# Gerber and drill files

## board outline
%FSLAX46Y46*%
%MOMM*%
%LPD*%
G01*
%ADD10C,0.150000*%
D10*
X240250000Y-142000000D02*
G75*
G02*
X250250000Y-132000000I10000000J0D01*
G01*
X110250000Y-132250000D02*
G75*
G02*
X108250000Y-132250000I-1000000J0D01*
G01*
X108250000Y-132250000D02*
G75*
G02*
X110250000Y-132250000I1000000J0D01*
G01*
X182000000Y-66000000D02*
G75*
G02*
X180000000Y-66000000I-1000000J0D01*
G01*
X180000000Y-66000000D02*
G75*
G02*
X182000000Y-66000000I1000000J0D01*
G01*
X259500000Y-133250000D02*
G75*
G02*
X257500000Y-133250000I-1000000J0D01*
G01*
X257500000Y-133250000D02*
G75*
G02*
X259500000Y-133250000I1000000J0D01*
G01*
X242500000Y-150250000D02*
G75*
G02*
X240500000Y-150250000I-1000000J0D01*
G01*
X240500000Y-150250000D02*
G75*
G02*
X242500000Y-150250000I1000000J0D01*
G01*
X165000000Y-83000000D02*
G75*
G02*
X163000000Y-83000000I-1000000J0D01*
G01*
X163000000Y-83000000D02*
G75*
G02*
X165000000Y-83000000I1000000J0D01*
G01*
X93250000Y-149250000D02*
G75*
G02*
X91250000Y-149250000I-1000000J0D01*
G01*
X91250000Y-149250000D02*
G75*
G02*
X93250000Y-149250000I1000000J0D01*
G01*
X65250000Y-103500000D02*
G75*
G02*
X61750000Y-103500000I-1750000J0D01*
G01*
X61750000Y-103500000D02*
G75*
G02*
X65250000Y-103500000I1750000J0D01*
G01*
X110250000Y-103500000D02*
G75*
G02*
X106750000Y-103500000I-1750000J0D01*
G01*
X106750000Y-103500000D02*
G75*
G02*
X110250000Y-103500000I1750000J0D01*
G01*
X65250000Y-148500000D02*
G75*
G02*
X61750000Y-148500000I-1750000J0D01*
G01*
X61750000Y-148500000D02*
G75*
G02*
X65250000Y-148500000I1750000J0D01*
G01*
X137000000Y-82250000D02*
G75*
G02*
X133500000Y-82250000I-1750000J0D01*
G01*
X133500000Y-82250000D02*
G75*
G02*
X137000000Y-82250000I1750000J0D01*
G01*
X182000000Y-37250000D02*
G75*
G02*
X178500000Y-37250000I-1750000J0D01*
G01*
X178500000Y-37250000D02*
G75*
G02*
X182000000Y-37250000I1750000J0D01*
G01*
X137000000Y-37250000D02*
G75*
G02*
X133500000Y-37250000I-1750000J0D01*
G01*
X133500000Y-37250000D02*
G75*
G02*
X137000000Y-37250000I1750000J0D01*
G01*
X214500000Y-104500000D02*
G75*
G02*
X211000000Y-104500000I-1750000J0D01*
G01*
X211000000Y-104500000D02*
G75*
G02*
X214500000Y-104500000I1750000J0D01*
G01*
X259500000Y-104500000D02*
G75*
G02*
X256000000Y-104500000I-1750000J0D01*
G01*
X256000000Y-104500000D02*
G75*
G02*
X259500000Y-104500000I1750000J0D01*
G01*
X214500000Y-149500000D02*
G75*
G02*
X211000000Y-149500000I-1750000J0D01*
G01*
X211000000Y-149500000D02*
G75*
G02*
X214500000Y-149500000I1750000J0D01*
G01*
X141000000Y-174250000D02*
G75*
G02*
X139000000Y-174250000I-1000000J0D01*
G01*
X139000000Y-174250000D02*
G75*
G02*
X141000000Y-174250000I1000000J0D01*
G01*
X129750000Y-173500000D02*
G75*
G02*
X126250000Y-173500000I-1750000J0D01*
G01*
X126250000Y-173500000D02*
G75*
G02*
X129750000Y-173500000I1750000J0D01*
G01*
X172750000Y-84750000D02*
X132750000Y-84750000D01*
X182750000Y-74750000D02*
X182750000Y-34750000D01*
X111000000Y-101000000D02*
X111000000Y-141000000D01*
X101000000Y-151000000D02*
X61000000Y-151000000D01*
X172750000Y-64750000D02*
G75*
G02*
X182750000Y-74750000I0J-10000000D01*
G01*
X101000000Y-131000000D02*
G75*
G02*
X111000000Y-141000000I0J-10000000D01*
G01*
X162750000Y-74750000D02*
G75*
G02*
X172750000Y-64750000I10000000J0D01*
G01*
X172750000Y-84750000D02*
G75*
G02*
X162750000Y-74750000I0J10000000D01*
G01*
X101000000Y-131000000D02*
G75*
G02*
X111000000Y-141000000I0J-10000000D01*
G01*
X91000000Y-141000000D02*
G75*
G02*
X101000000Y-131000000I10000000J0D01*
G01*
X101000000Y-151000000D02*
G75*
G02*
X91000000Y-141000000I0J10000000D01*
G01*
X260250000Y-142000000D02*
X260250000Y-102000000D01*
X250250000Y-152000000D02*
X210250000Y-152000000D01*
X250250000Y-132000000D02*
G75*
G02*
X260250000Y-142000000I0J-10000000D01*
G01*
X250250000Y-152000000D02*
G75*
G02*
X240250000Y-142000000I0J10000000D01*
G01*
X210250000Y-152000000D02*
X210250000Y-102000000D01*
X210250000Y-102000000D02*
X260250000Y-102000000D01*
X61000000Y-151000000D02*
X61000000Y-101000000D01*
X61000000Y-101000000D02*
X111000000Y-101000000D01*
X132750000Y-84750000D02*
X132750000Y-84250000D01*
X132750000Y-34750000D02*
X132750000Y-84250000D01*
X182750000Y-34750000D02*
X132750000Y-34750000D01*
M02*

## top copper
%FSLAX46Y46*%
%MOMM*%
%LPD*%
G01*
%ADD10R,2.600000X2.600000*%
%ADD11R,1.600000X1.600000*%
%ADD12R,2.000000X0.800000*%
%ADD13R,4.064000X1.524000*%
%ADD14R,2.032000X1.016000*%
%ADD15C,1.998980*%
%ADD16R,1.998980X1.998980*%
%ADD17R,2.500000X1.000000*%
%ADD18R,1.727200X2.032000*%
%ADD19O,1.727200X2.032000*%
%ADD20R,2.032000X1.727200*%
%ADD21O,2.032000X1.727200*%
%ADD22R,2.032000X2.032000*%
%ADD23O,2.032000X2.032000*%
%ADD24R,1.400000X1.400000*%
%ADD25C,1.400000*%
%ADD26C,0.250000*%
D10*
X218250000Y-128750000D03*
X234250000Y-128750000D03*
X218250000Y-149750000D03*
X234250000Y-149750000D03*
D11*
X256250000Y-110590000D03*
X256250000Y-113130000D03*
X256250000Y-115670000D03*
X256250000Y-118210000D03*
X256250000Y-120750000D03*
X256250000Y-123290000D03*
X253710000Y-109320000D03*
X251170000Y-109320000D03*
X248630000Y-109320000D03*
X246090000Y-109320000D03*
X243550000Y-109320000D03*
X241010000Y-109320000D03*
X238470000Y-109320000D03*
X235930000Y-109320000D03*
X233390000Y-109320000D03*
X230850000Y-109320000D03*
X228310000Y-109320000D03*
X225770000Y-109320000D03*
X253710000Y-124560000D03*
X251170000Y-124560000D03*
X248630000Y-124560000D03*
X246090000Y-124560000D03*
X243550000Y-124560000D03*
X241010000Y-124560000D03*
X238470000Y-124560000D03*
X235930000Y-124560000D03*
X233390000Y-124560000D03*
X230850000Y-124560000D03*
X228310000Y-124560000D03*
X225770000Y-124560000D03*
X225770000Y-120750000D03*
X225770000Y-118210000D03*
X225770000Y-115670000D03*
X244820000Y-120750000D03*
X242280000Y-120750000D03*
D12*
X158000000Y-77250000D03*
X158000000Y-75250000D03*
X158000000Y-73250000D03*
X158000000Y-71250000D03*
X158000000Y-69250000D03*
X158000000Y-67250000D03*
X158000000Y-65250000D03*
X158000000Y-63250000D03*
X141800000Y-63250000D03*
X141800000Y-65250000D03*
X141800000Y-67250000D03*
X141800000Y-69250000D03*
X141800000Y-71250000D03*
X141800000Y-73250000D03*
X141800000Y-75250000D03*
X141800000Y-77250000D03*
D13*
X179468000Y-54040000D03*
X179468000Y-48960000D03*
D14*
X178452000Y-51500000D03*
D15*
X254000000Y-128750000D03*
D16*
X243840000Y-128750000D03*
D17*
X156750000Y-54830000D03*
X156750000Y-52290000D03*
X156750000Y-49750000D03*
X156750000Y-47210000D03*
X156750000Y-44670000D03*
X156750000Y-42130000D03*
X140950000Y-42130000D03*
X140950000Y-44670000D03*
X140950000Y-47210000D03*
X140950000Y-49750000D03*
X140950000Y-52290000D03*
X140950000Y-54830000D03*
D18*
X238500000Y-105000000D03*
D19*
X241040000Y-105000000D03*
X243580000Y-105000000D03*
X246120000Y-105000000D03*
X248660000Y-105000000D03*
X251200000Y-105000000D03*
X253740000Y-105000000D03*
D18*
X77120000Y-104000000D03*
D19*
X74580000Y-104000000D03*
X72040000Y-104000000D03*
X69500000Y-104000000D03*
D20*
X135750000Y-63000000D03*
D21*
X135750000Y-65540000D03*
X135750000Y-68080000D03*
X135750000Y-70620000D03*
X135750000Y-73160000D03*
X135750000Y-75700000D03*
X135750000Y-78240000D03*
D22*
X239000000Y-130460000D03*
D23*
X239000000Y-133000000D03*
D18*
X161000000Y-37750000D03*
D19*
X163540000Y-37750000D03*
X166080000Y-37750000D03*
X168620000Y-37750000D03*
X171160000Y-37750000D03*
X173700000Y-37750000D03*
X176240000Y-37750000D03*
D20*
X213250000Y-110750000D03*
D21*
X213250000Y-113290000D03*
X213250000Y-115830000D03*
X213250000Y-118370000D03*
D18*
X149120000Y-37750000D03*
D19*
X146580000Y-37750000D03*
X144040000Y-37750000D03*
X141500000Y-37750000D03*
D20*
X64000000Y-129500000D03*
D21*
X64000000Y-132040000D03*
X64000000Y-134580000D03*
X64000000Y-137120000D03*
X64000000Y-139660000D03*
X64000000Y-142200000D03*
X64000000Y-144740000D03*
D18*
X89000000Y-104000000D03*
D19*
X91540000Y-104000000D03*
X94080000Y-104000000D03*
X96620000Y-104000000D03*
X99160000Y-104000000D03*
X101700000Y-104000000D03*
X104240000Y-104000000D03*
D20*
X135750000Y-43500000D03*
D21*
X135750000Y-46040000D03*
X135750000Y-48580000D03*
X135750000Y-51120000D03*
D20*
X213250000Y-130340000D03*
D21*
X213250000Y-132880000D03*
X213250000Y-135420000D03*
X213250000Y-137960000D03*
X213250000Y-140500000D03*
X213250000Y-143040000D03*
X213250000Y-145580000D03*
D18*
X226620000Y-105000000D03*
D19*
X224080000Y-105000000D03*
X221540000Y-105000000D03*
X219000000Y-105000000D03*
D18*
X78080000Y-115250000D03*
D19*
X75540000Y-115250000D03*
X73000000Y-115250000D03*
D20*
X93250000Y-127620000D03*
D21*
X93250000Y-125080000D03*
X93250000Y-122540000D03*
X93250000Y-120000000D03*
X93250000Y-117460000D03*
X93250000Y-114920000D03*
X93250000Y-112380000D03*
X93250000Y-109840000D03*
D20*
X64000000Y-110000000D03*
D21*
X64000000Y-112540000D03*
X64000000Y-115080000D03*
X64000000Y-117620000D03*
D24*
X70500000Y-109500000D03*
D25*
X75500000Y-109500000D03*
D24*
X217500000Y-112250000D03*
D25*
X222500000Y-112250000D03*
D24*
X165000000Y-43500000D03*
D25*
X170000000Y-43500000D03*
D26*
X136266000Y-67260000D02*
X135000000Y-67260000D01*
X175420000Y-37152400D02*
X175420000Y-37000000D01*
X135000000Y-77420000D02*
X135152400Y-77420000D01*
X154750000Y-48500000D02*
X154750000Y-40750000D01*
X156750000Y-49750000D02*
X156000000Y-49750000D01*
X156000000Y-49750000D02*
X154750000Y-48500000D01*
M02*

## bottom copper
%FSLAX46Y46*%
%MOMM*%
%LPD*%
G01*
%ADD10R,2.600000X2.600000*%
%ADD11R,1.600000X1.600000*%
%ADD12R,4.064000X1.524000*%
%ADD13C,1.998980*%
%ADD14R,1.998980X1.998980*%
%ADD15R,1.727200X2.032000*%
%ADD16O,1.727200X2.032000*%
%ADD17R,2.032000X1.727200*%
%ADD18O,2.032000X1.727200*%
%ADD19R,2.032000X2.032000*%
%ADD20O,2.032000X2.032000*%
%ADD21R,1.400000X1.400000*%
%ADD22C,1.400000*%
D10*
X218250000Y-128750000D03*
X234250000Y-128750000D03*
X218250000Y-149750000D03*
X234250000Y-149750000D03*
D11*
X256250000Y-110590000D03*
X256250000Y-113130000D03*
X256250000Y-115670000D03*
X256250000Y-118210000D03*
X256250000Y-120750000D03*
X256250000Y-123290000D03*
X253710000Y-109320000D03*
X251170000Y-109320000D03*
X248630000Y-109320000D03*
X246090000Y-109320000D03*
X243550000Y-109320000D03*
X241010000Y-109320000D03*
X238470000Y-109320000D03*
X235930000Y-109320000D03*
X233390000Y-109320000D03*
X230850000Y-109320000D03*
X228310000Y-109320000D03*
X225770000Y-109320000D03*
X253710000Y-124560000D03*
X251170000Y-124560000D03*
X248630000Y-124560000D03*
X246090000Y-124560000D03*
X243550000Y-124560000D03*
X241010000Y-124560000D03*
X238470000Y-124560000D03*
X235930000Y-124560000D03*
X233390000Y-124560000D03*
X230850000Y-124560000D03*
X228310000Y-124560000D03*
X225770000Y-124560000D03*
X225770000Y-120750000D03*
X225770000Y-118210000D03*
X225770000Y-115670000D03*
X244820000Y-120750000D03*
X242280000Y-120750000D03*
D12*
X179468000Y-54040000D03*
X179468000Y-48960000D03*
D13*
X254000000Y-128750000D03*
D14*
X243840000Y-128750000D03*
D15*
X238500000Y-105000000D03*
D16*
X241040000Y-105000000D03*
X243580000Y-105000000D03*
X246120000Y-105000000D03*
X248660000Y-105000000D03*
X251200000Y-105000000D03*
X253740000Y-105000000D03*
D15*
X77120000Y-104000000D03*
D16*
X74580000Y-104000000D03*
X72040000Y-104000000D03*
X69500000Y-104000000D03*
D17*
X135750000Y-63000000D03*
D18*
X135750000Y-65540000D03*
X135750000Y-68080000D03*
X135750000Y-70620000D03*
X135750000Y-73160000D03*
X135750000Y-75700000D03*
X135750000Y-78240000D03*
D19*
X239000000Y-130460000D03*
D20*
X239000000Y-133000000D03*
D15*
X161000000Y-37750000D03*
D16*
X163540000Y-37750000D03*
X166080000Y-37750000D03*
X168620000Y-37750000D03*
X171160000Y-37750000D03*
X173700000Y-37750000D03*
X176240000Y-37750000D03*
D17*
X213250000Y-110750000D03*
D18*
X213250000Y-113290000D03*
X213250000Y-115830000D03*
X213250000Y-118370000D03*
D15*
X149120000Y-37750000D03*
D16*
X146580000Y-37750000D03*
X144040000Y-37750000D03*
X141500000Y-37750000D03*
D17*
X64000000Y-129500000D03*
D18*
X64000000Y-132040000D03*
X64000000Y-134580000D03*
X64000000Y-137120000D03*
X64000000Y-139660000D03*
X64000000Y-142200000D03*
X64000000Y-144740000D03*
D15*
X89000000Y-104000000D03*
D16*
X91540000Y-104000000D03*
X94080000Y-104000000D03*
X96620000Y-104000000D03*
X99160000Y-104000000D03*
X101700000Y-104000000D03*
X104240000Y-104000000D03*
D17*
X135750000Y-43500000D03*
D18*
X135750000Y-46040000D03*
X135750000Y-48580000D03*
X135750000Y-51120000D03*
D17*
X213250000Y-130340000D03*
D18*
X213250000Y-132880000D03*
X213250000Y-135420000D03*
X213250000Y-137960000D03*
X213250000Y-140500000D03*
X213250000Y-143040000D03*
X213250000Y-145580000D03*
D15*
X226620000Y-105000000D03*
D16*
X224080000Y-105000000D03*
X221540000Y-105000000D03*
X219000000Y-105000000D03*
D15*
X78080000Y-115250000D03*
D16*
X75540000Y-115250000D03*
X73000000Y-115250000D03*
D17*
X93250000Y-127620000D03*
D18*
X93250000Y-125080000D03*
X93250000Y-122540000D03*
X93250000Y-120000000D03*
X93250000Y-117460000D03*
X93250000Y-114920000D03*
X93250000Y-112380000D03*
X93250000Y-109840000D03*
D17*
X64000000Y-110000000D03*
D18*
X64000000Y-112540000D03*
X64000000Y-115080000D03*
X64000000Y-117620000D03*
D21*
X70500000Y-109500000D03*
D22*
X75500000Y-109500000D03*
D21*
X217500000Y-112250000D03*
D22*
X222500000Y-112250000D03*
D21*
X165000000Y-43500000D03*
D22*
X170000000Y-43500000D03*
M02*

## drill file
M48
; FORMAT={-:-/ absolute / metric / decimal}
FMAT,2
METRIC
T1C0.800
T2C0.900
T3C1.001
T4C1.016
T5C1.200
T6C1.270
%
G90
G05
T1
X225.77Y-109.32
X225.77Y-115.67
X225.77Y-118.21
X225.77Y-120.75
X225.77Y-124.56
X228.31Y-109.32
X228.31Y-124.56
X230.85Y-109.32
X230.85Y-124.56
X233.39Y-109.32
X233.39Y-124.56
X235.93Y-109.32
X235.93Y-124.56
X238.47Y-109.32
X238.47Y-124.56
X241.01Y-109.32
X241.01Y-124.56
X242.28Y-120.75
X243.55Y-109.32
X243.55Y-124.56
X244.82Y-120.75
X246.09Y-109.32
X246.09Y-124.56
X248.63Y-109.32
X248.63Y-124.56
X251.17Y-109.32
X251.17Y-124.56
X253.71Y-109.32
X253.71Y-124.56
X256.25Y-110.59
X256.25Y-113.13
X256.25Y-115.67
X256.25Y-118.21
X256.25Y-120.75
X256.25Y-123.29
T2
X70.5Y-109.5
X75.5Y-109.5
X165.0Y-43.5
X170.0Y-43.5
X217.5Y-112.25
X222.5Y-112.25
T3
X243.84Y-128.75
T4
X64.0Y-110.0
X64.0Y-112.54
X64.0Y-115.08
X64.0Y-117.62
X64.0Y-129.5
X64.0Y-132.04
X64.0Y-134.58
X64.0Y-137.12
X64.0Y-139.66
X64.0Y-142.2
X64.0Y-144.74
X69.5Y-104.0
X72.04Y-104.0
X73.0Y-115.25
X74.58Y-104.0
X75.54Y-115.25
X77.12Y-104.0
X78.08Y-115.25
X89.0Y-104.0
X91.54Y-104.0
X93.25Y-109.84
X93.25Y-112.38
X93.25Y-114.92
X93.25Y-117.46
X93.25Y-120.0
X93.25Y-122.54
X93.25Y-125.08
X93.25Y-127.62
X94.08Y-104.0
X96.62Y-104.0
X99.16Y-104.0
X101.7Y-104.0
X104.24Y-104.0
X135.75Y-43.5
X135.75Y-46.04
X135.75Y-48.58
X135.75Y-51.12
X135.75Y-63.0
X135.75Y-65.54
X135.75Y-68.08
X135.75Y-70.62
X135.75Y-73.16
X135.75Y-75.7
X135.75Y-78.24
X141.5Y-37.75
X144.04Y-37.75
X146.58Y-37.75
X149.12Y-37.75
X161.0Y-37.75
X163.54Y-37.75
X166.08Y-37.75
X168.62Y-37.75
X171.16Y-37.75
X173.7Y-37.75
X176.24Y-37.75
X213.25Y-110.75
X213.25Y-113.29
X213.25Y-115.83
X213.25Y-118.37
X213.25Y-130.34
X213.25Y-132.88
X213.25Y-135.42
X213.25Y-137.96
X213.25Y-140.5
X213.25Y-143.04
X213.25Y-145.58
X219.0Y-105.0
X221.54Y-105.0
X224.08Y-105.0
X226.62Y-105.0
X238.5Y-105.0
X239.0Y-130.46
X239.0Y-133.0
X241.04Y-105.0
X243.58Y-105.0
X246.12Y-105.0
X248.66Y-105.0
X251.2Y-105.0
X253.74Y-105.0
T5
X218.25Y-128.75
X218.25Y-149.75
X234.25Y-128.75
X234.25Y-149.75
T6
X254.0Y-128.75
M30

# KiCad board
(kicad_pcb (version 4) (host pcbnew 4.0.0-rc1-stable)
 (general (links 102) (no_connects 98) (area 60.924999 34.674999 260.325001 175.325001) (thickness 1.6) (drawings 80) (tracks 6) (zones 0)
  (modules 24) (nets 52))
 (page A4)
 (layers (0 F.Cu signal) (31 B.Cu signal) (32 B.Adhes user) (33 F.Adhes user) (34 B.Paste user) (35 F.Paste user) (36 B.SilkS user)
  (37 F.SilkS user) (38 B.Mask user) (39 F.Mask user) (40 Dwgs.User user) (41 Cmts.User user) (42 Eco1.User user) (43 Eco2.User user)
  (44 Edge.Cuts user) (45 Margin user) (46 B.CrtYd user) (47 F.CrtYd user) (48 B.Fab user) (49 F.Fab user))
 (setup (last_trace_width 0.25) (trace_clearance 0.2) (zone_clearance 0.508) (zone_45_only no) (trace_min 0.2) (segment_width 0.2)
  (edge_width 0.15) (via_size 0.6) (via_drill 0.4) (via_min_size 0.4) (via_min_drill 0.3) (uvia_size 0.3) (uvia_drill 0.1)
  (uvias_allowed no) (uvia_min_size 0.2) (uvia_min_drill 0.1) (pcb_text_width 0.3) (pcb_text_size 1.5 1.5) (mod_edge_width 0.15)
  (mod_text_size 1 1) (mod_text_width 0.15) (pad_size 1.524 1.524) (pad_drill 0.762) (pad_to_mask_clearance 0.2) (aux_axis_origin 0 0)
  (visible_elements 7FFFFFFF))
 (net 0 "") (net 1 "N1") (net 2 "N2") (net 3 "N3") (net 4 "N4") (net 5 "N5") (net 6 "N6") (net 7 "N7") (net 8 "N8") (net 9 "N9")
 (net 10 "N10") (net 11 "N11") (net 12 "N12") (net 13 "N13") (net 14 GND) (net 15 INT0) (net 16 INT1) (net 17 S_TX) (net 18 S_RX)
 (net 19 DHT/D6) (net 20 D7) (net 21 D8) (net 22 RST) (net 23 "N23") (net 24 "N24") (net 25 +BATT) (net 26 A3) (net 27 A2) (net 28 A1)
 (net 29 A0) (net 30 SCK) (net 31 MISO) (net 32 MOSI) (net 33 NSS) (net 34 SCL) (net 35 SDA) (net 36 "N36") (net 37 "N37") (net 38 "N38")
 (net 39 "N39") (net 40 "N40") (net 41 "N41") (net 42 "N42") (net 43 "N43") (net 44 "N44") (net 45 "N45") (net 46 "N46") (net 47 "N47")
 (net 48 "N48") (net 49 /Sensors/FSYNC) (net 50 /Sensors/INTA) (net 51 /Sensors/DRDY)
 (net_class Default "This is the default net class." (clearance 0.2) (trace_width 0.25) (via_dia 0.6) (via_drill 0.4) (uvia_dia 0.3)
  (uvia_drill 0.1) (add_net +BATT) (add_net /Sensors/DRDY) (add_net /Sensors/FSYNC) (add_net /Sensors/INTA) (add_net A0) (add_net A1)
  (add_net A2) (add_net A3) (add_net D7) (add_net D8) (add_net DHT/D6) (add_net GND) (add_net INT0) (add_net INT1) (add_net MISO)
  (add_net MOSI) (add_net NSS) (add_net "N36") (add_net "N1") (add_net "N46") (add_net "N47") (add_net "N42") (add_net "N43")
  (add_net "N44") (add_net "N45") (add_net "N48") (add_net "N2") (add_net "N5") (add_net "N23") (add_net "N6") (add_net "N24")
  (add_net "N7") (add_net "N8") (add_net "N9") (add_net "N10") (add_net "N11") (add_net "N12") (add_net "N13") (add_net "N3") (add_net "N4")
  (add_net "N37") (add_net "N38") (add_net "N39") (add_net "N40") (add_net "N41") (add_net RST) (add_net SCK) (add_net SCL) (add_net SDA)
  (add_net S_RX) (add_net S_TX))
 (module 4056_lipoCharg (layer F.Cu) (at 215.5 125.5)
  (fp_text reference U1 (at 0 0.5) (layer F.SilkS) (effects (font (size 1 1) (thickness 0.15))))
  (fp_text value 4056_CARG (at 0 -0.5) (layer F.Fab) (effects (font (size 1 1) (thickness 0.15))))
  (pad 3 thru_hole rect (at 2.75 3.25) (size 2.6 2.6) (drill 1.2) (layers *.Cu *.Mask F.SilkS) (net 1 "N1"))
  (pad 4 thru_hole rect (at 18.75 3.25) (size 2.6 2.6) (drill 1.2) (layers *.Cu *.Mask F.SilkS) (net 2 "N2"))
  (pad 1 thru_hole rect (at 2.75 24.25) (size 2.6 2.6) (drill 1.2) (layers *.Cu *.Mask F.SilkS) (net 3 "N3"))
  (pad 2 thru_hole rect (at 18.75 24.25) (size 2.6 2.6) (drill 1.2) (layers *.Cu *.Mask F.SilkS) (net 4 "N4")))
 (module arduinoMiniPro (layer F.Cu) (at 247.36 114.4 270)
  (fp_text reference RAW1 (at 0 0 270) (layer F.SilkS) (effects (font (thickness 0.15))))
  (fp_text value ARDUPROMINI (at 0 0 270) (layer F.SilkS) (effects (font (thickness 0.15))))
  (pad 1 thru_hole rect (at -3.81 -8.89) (size 1.6 1.6) (drill 0.8) (layers *.Cu *.Mask) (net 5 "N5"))
  (pad 2 thru_hole rect (at -1.27 -8.89) (size 1.6 1.6) (drill 0.8) (layers *.Cu *.Mask) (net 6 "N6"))
  (pad 3 thru_hole rect (at 1.27 -8.89) (size 1.6 1.6) (drill 0.8) (layers *.Cu *.Mask) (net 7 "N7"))
  (pad 4 thru_hole rect (at 3.81 -8.89) (size 1.6 1.6) (drill 0.8) (layers *.Cu *.Mask) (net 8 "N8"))
  (pad 5 thru_hole rect (at 6.35 -8.89) (size 1.6 1.6) (drill 0.8) (layers *.Cu *.Mask) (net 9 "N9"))
  (pad 6 thru_hole rect (at 8.89 -8.89) (size 1.6 1.6) (drill 0.8) (layers *.Cu *.Mask) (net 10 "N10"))
  (pad 7 thru_hole rect (at -5.08 -6.35 90) (size 1.6 1.6) (drill 0.8) (layers *.Cu *.Mask) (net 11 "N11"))
  (pad 8 thru_hole rect (at -5.08 -3.81 90) (size 1.6 1.6) (drill 0.8) (layers *.Cu *.Mask) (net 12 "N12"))
  (pad 9 thru_hole rect (at -5.08 -1.27 90) (size 1.6 1.6) (drill 0.8) (layers *.Cu *.Mask) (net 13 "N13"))
  (pad 10 thru_hole rect (at -5.08 1.27 90) (size 1.6 1.6) (drill 0.8) (layers *.Cu *.Mask) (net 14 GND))
  (pad 11 thru_hole rect (at -5.08 3.81 90) (size 1.6 1.6) (drill 0.8) (layers *.Cu *.Mask) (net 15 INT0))
  (pad 12 thru_hole rect (at -5.08 6.35 90) (size 1.6 1.6) (drill 0.8) (layers *.Cu *.Mask) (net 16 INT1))
  (pad 13 thru_hole rect (at -5.08 8.89 90) (size 1.6 1.6) (drill 0.8) (layers *.Cu *.Mask) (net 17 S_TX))
  (pad 14 thru_hole rect (at -5.08 11.43 90) (size 1.6 1.6) (drill 0.8) (layers *.Cu *.Mask) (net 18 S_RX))
  (pad 15 thru_hole rect (at -5.08 13.97 90) (size 1.6 1.6) (drill 0.8) (layers *.Cu *.Mask) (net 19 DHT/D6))
  (pad 16 thru_hole rect (at -5.08 16.51 90) (size 1.6 1.6) (drill 0.8) (layers *.Cu *.Mask) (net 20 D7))
  (pad 17 thru_hole rect (at -5.08 19.05 90) (size 1.6 1.6) (drill 0.8) (layers *.Cu *.Mask) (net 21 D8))
  (pad 18 thru_hole rect (at -5.08 21.59 90) (size 1.6 1.6) (drill 0.8) (layers *.Cu *.Mask) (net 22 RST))
  (pad 19 thru_hole rect (at 10.16 -6.35 90) (size 1.6 1.6) (drill 0.8) (layers *.Cu *.Mask) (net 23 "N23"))
  (pad 20 thru_hole rect (at 10.16 -3.81 90) (size 1.6 1.6) (drill 0.8) (layers *.Cu *.Mask) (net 14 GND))
  (pad 21 thru_hole rect (at 10.16 -1.27 90) (size 1.6 1.6) (drill 0.8) (layers *.Cu *.Mask) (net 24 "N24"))
  (pad 22 thru_hole rect (at 10.16 1.27 90) (size 1.6 1.6) (drill 0.8) (layers *.Cu *.Mask) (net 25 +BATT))
  (pad 23 thru_hole rect (at 10.16 3.81 90) (size 1.6 1.6) (drill 0.8) (layers *.Cu *.Mask) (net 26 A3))
  (pad 24 thru_hole rect (at 10.16 6.35 90) (size 1.6 1.6) (drill 0.8) (layers *.Cu *.Mask) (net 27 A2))
  (pad 25 thru_hole rect (at 10.16 8.89 90) (size 1.6 1.6) (drill 0.8) (layers *.Cu *.Mask) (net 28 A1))
  (pad 26 thru_hole rect (at 10.16 11.43 90) (size 1.6 1.6) (drill 0.8) (layers *.Cu *.Mask) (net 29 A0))
  (pad 27 thru_hole rect (at 10.16 13.97 90) (size 1.6 1.6) (drill 0.8) (layers *.Cu *.Mask) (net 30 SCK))
  (pad 28 thru_hole rect (at 10.16 16.51 90) (size 1.6 1.6) (drill 0.8) (layers *.Cu *.Mask) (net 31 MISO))
  (pad 29 thru_hole rect (at 10.16 19.05 90) (size 1.6 1.6) (drill 0.8) (layers *.Cu *.Mask) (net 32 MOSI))
  (pad 30 thru_hole rect (at 10.16 21.59 90) (size 1.6 1.6) (drill 0.8) (layers *.Cu *.Mask) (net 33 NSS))
  (pad A7 thru_hole rect (at 6.35 21.59 180) (size 1.6 1.6) (drill 0.8) (layers *.Cu *.Mask))
  (pad A6 thru_hole rect (at 3.81 21.59 180) (size 1.6 1.6) (drill 0.8) (layers *.Cu *.Mask))
  (pad GND4 thru_hole rect (at 1.27 21.59 180) (size 1.6 1.6) (drill 0.8) (layers *.Cu *.Mask))
  (pad 32 thru_hole rect (at 6.35 2.54 180) (size 1.6 1.6) (drill 0.8) (layers *.Cu *.Mask) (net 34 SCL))
  (pad 31 thru_hole rect (at 6.35 5.08 180) (size 1.6 1.6) (drill 0.8) (layers *.Cu *.Mask) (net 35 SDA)))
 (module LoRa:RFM (layer F.Cu) (at 149.9 70.25)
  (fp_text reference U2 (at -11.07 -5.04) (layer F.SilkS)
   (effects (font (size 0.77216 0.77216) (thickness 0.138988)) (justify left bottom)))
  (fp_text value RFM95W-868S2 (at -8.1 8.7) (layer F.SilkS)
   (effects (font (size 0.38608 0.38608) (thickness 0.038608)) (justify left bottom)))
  (pad 9 smd rect (at 8.1 7 180) (size 2 0.8) (layers F.Cu F.Paste F.Mask) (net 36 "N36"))
  (pad 10 smd rect (at 8.1 5 180) (size 2 0.8) (layers F.Cu F.Paste F.Mask) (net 14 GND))
  (pad 11 smd rect (at 8.1 3 180) (size 2 0.8) (layers F.Cu F.Paste F.Mask) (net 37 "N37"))
  (pad 12 smd rect (at 8.1 1 180) (size 2 0.8) (layers F.Cu F.Paste F.Mask) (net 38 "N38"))
  (pad 13 smd rect (at 8.1 -1 180) (size 2 0.8) (layers F.Cu F.Paste F.Mask) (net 25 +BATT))
  (pad 14 smd rect (at 8.1 -3 180) (size 2 0.8) (layers F.Cu F.Paste F.Mask) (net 15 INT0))
  (pad 15 smd rect (at 8.1 -5 180) (size 2 0.8) (layers F.Cu F.Paste F.Mask) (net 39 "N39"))
  (pad 16 smd rect (at 8.1 -7 180) (size 2 0.8) (layers F.Cu F.Paste F.Mask) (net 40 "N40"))
  (pad 1 smd rect (at -8.1 -7) (size 2 0.8) (layers F.Cu F.Paste F.Mask) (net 14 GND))
  (pad 2 smd rect (at -8.1 -5) (size 2 0.8) (layers F.Cu F.Paste F.Mask) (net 31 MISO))
  (pad 3 smd rect (at -8.1 -3) (size 2 0.8) (layers F.Cu F.Paste F.Mask) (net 32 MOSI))
  (pad 4 smd rect (at -8.1 -1) (size 2 0.8) (layers F.Cu F.Paste F.Mask) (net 30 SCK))
  (pad 5 smd rect (at -8.1 1) (size 2 0.8) (layers F.Cu F.Paste F.Mask) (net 33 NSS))
  (pad 6 smd rect (at -8.1 3) (size 2 0.8) (layers F.Cu F.Paste F.Mask) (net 22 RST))
  (pad 7 smd rect (at -8.1 5) (size 2 0.8) (layers F.Cu F.Paste F.Mask) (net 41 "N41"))
  (pad 8 smd rect (at -8.1 7 180) (size 2 0.8) (layers F.Cu F.Paste F.Mask) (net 14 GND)))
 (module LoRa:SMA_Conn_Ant (layer F.Cu) (at 181.5 51.5 180)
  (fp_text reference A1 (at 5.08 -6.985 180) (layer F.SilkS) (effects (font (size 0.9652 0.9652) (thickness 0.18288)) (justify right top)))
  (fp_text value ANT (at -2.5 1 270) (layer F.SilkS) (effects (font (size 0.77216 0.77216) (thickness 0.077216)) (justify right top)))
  (pad 1 smd rect (at 2.032 -2.54 270) (size 1.524 4.064) (layers F.Cu F.Paste F.Mask) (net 14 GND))
  (pad 3 smd rect (at 2.032 2.54 270) (size 1.524 4.064) (layers F.Cu F.Paste F.Mask) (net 14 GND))
  (pad 2 smd rect (at 3.048 0 270) (size 1.016 2.032) (layers F.Cu F.Paste F.Mask) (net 36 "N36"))
  (pad "" smd rect (at 2.032 -2.54 270) (size 1.524 4.064) (layers B.Cu B.Paste B.Mask))
  (pad "" smd rect (at 2.032 2.54 270) (size 1.524 4.064) (layers B.Cu B.Paste B.Mask)))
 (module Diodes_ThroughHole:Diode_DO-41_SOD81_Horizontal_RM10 (layer F.Cu) (at 243.84 128.75254)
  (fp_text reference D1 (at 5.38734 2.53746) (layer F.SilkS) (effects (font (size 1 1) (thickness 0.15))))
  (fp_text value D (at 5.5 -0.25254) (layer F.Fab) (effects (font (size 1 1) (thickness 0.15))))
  (pad 2 thru_hole circle (at 10.16 -0.00254 180) (size 1.99898 1.99898) (drill 1.27) (layers *.Cu *.Mask F.SilkS) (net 1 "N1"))
  (pad 1 thru_hole rect (at 0 -0.00254 180) (size 1.99898 1.99898) (drill 1.00076) (layers *.Cu *.Mask F.SilkS) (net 25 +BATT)))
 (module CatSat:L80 (layer F.Cu) (at 148.883668 49.118506 180) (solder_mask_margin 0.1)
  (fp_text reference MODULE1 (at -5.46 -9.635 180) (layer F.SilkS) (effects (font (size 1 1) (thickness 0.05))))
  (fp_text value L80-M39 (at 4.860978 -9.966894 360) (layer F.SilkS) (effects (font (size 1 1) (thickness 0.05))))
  (pad 1 smd rect (at -7.866332 -5.711494) (size 2.5 1) (layers F.Cu F.Paste F.Mask) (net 17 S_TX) (solder_mask_margin 0.2))
  (pad 2 smd rect (at -7.866332 -3.171494) (size 2.5 1) (layers F.Cu F.Paste F.Mask) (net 18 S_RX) (solder_mask_margin 0.2))
  (pad 3 smd rect (at -7.866332 -0.631494) (size 2.5 1) (layers F.Cu F.Paste F.Mask) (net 14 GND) (solder_mask_margin 0.2))
  (pad 4 smd rect (at -7.866332 1.908506) (size 2.5 1) (layers F.Cu F.Paste F.Mask) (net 25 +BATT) (solder_mask_margin 0.2))
  (pad 5 smd rect (at -7.866332 4.448506) (size 2.5 1) (layers F.Cu F.Paste F.Mask) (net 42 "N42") (solder_mask_margin 0.2))
  (pad 6 smd rect (at -7.866332 6.988506) (size 2.5 1) (layers F.Cu F.Paste F.Mask) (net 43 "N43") (solder_mask_margin 0.2))
  (pad 7 smd rect (at 7.933668 6.988506 180) (size 2.5 1) (layers F.Cu F.Paste F.Mask) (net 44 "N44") (solder_mask_margin 0.2))
  (pad 8 smd rect (at 7.933668 4.448506 180) (size 2.5 1) (layers F.Cu F.Paste F.Mask) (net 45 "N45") (solder_mask_margin 0.2))
  (pad 9 smd rect (at 7.933668 1.908506 180) (size 2.5 1) (layers F.Cu F.Paste F.Mask) (solder_mask_margin 0.2))
  (pad 10 smd rect (at 7.933668 -0.631494 180) (size 2.5 1) (layers F.Cu F.Paste F.Mask) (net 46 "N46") (solder_mask_margin 0.2))
  (pad 11 smd rect (at 7.933668 -3.171494 180) (size 2.5 1) (layers F.Cu F.Paste F.Mask) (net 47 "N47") (solder_mask_margin 0.2))
  (pad 12 smd rect (at 7.933668 -5.711494) (size 2.5 1) (layers F.Cu F.Paste F.Mask) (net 14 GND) (solder_mask_margin 0.2)))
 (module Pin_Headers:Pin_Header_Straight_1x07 (layer F.Cu) (at 238.5 105 90)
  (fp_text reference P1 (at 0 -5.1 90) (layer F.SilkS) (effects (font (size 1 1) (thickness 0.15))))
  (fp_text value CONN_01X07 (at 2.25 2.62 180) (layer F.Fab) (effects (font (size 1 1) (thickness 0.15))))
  (pad 1 thru_hole rect (at 0 0 90) (size 2.032 1.7272) (drill 1.016) (layers *.Cu *.Mask F.SilkS) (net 14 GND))
  (pad 2 thru_hole oval (at 0 2.54 90) (size 2.032 1.7272) (drill 1.016) (layers *.Cu *.Mask F.SilkS) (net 25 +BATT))
  (pad 3 thru_hole oval (at 0 5.08 90) (size 2.032 1.7272) (drill 1.016) (layers *.Cu *.Mask F.SilkS) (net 34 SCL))
  (pad 4 thru_hole oval (at 0 7.62 90) (size 2.032 1.7272) (drill 1.016) (layers *.Cu *.Mask F.SilkS) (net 35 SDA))
  (pad 5 thru_hole oval (at 0 10.16 90) (size 2.032 1.7272) (drill 1.016) (layers *.Cu *.Mask F.SilkS) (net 18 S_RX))
  (pad 6 thru_hole oval (at 0 12.7 90) (size 2.032 1.7272) (drill 1.016) (layers *.Cu *.Mask F.SilkS) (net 17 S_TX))
  (pad 7 thru_hole oval (at 0 15.24 90) (size 2.032 1.7272) (drill 1.016) (layers *.Cu *.Mask F.SilkS) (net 19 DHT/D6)))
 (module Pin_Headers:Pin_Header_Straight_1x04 (layer F.Cu) (at 77.12 104 270)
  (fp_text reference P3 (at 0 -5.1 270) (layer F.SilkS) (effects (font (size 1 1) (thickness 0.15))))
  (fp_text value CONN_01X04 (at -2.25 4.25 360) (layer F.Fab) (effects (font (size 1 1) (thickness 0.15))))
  (pad 1 thru_hole rect (at 0 0 270) (size 2.032 1.7272) (drill 1.016) (layers *.Cu *.Mask F.SilkS) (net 15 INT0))
  (pad 2 thru_hole oval (at 0 2.54 270) (size 2.032 1.7272) (drill 1.016) (layers *.Cu *.Mask F.SilkS) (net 16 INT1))
  (pad 3 thru_hole oval (at 0 5.08 270) (size 2.032 1.7272) (drill 1.016) (layers *.Cu *.Mask F.SilkS) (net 20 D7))
  (pad 4 thru_hole oval (at 0 7.62 270) (size 2.032 1.7272) (drill 1.016) (layers *.Cu *.Mask F.SilkS) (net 21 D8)))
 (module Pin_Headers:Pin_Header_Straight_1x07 (layer F.Cu) (at 135.75 63)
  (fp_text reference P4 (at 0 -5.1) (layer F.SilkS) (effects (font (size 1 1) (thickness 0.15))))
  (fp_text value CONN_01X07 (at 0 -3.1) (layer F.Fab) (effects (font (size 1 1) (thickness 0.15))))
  (pad 1 thru_hole rect (at 0 0) (size 2.032 1.7272) (drill 1.016) (layers *.Cu *.Mask F.SilkS) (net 25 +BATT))
  (pad 2 thru_hole oval (at 0 2.54) (size 2.032 1.7272) (drill 1.016) (layers *.Cu *.Mask F.SilkS) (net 14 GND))
  (pad 3 thru_hole oval (at 0 5.08) (size 2.032 1.7272) (drill 1.016) (layers *.Cu *.Mask F.SilkS) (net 30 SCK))
  (pad 4 thru_hole oval (at 0 7.62) (size 2.032 1.7272) (drill 1.016) (layers *.Cu *.Mask F.SilkS) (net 31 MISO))
  (pad 5 thru_hole oval (at 0 10.16) (size 2.032 1.7272) (drill 1.016) (layers *.Cu *.Mask F.SilkS) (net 32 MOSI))
  (pad 6 thru_hole oval (at 0 12.7) (size 2.032 1.7272) (drill 1.016) (layers *.Cu *.Mask F.SilkS) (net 33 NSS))
  (pad 7 thru_hole oval (at 0 15.24) (size 2.032 1.7272) (drill 1.016) (layers *.Cu *.Mask F.SilkS) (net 22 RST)))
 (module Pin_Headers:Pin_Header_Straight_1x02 (layer F.Cu) (at 239 130.46)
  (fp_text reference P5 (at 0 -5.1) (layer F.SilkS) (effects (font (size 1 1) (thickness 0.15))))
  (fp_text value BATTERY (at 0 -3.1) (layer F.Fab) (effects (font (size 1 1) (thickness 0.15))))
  (pad 1 thru_hole rect (at 0 0) (size 2.032 2.032) (drill 1.016) (layers *.Cu *.Mask F.SilkS) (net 1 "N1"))
  (pad 2 thru_hole oval (at 0 2.54) (size 2.032 2.032) (drill 1.016) (layers *.Cu *.Mask F.SilkS) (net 2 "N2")))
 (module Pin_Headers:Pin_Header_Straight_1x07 (layer F.Cu) (at 161 37.75 90)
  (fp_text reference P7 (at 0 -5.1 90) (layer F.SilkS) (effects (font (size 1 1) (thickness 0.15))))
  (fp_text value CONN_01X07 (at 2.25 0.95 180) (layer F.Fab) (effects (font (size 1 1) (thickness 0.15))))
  (pad 1 thru_hole rect (at 0 0 90) (size 2.032 1.7272) (drill 1.016) (layers *.Cu *.Mask F.SilkS) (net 14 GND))
  (pad 2 thru_hole oval (at 0 2.54 90) (size 2.032 1.7272) (drill 1.016) (layers *.Cu *.Mask F.SilkS) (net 25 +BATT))
  (pad 3 thru_hole oval (at 0 5.08 90) (size 2.032 1.7272) (drill 1.016) (layers *.Cu *.Mask F.SilkS) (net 34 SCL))
  (pad 4 thru_hole oval (at 0 7.62 90) (size 2.032 1.7272) (drill 1.016) (layers *.Cu *.Mask F.SilkS) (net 35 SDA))
  (pad 5 thru_hole oval (at 0 10.16 90) (size 2.032 1.7272) (drill 1.016) (layers *.Cu *.Mask F.SilkS) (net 18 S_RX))
  (pad 6 thru_hole oval (at 0 12.7 90) (size 2.032 1.7272) (drill 1.016) (layers *.Cu *.Mask F.SilkS) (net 17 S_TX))
  (pad 7 thru_hole oval (at 0 15.24 90) (size 2.032 1.7272) (drill 1.016) (layers *.Cu *.Mask F.SilkS) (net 19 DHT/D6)))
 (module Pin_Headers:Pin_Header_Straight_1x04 (layer F.Cu) (at 213.25 110.75)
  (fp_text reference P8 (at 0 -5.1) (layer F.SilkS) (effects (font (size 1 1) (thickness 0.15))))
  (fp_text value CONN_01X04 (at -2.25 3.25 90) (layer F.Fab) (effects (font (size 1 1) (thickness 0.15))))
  (pad 1 thru_hole rect (at 0 0) (size 2.032 1.7272) (drill 1.016) (layers *.Cu *.Mask F.SilkS) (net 26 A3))
  (pad 2 thru_hole oval (at 0 2.54) (size 2.032 1.7272) (drill 1.016) (layers *.Cu *.Mask F.SilkS) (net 27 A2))
  (pad 3 thru_hole oval (at 0 5.08) (size 2.032 1.7272) (drill 1.016) (layers *.Cu *.Mask F.SilkS) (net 28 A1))
  (pad 4 thru_hole oval (at 0 7.62) (size 2.032 1.7272) (drill 1.016) (layers *.Cu *.Mask F.SilkS) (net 29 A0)))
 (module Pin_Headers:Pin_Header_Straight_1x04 (layer F.Cu) (at 149.12 37.75 270)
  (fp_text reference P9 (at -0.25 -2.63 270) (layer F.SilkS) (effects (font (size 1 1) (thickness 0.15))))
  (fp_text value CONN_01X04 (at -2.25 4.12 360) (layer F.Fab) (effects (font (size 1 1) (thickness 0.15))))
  (pad 1 thru_hole rect (at 0 0 270) (size 2.032 1.7272) (drill 1.016) (layers *.Cu *.Mask F.SilkS) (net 15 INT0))
  (pad 2 thru_hole oval (at 0 2.54 270) (size 2.032 1.7272) (drill 1.016) (layers *.Cu *.Mask F.SilkS) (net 16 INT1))
  (pad 3 thru_hole oval (at 0 5.08 270) (size 2.032 1.7272) (drill 1.016) (layers *.Cu *.Mask F.SilkS) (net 20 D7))
  (pad 4 thru_hole oval (at 0 7.62 270) (size 2.032 1.7272) (drill 1.016) (layers *.Cu *.Mask F.SilkS) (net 21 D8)))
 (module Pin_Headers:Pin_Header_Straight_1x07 (layer F.Cu) (at 64 129.5)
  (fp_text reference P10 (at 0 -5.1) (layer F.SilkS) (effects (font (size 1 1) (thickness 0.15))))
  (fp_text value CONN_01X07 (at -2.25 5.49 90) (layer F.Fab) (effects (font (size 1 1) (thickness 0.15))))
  (pad 1 thru_hole rect (at 0 0) (size 2.032 1.7272) (drill 1.016) (layers *.Cu *.Mask F.SilkS) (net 25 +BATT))
  (pad 2 thru_hole oval (at 0 2.54) (size 2.032 1.7272) (drill 1.016) (layers *.Cu *.Mask F.SilkS) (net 14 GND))
  (pad 3 thru_hole oval (at 0 5.08) (size 2.032 1.7272) (drill 1.016) (layers *.Cu *.Mask F.SilkS) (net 30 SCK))
  (pad 4 thru_hole oval (at 0 7.62) (size 2.032 1.7272) (drill 1.016) (layers *.Cu *.Mask F.SilkS) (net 31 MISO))
  (pad 5 thru_hole oval (at 0 10.16) (size 2.032 1.7272) (drill 1.016) (layers *.Cu *.Mask F.SilkS) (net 32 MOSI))
  (pad 6 thru_hole oval (at 0 12.7) (size 2.032 1.7272) (drill 1.016) (layers *.Cu *.Mask F.SilkS) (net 33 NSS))
  (pad 7 thru_hole oval (at 0 15.24) (size 2.032 1.7272) (drill 1.016) (layers *.Cu *.Mask F.SilkS) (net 22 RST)))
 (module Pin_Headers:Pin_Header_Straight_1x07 (layer F.Cu) (at 89 104 90)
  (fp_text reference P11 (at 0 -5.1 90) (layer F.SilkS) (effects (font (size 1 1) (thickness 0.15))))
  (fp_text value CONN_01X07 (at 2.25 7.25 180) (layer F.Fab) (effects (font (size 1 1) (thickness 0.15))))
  (pad 1 thru_hole rect (at 0 0 90) (size 2.032 1.7272) (drill 1.016) (layers *.Cu *.Mask F.SilkS) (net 14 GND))
  (pad 2 thru_hole oval (at 0 2.54 90) (size 2.032 1.7272) (drill 1.016) (layers *.Cu *.Mask F.SilkS) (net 25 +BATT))
  (pad 3 thru_hole oval (at 0 5.08 90) (size 2.032 1.7272) (drill 1.016) (layers *.Cu *.Mask F.SilkS) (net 34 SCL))
  (pad 4 thru_hole oval (at 0 7.62 90) (size 2.032 1.7272) (drill 1.016) (layers *.Cu *.Mask F.SilkS) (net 35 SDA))
  (pad 5 thru_hole oval (at 0 10.16 90) (size 2.032 1.7272) (drill 1.016) (layers *.Cu *.Mask F.SilkS) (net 18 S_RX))
  (pad 6 thru_hole oval (at 0 12.7 90) (size 2.032 1.7272) (drill 1.016) (layers *.Cu *.Mask F.SilkS) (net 17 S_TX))
  (pad 7 thru_hole oval (at 0 15.24 90) (size 2.032 1.7272) (drill 1.016) (layers *.Cu *.Mask F.SilkS) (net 19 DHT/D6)))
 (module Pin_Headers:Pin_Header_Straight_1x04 (layer F.Cu) (at 135.75 43.5)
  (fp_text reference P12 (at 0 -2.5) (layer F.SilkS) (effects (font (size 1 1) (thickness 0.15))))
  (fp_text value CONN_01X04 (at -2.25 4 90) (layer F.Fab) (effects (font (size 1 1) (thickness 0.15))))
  (pad 1 thru_hole rect (at 0 0) (size 2.032 1.7272) (drill 1.016) (layers *.Cu *.Mask F.SilkS) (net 26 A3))
  (pad 2 thru_hole oval (at 0 2.54) (size 2.032 1.7272) (drill 1.016) (layers *.Cu *.Mask F.SilkS) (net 27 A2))
  (pad 3 thru_hole oval (at 0 5.08) (size 2.032 1.7272) (drill 1.016) (layers *.Cu *.Mask F.SilkS) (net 28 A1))
  (pad 4 thru_hole oval (at 0 7.62) (size 2.032 1.7272) (drill 1.016) (layers *.Cu *.Mask F.SilkS) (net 29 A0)))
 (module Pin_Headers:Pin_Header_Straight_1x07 (layer F.Cu) (at 213.25 130.34)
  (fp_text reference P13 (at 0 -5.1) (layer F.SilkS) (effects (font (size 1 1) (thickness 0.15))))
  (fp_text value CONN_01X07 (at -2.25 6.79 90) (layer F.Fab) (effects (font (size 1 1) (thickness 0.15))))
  (pad 1 thru_hole rect (at 0 0) (size 2.032 1.7272) (drill 1.016) (layers *.Cu *.Mask F.SilkS) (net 25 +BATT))
  (pad 2 thru_hole oval (at 0 2.54) (size 2.032 1.7272) (drill 1.016) (layers *.Cu *.Mask F.SilkS) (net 14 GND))
  (pad 3 thru_hole oval (at 0 5.08) (size 2.032 1.7272) (drill 1.016) (layers *.Cu *.Mask F.SilkS) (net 30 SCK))
  (pad 4 thru_hole oval (at 0 7.62) (size 2.032 1.7272) (drill 1.016) (layers *.Cu *.Mask F.SilkS) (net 31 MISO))
  (pad 5 thru_hole oval (at 0 10.16) (size 2.032 1.7272) (drill 1.016) (layers *.Cu *.Mask F.SilkS) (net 32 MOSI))
  (pad 6 thru_hole oval (at 0 12.7) (size 2.032 1.7272) (drill 1.016) (layers *.Cu *.Mask F.SilkS) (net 33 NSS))
  (pad 7 thru_hole oval (at 0 15.24) (size 2.032 1.7272) (drill 1.016) (layers *.Cu *.Mask F.SilkS) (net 22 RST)))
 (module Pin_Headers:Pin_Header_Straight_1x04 (layer F.Cu) (at 226.62 105 270)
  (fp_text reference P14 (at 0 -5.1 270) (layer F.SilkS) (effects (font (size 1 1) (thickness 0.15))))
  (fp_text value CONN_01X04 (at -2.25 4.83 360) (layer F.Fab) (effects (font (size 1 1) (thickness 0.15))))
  (pad 1 thru_hole rect (at 0 0 270) (size 2.032 1.7272) (drill 1.016) (layers *.Cu *.Mask F.SilkS) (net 15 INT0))
  (pad 2 thru_hole oval (at 0 2.54 270) (size 2.032 1.7272) (drill 1.016) (layers *.Cu *.Mask F.SilkS) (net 16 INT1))
  (pad 3 thru_hole oval (at 0 5.08 270) (size 2.032 1.7272) (drill 1.016) (layers *.Cu *.Mask F.SilkS) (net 20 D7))
  (pad 4 thru_hole oval (at 0 7.62 270) (size 2.032 1.7272) (drill 1.016) (layers *.Cu *.Mask F.SilkS) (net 21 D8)))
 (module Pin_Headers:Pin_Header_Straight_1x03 (layer F.Cu) (at 78.08 115.25 270)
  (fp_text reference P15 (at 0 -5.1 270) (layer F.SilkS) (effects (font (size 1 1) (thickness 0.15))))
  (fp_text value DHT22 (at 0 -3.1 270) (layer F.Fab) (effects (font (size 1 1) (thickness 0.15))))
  (pad 1 thru_hole rect (at 0 0 270) (size 2.032 1.7272) (drill 1.016) (layers *.Cu *.Mask F.SilkS) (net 19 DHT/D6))
  (pad 2 thru_hole oval (at 0 2.54 270) (size 2.032 1.7272) (drill 1.016) (layers *.Cu *.Mask F.SilkS) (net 25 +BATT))
  (pad 3 thru_hole oval (at 0 5.08 270) (size 2.032 1.7272) (drill 1.016) (layers *.Cu *.Mask F.SilkS) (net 14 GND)))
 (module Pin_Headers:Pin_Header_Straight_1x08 (layer F.Cu) (at 93.25 127.62 180)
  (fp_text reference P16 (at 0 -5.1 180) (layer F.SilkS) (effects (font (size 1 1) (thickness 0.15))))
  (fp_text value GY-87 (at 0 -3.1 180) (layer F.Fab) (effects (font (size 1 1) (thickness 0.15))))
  (pad 1 thru_hole rect (at 0 0 180) (size 2.032 1.7272) (drill 1.016) (layers *.Cu *.Mask F.SilkS) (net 25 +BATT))
  (pad 2 thru_hole oval (at 0 2.54 180) (size 2.032 1.7272) (drill 1.016) (layers *.Cu *.Mask F.SilkS) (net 14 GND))
  (pad 3 thru_hole oval (at 0 5.08 180) (size 2.032 1.7272) (drill 1.016) (layers *.Cu *.Mask F.SilkS) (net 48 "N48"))
  (pad 4 thru_hole oval (at 0 7.62 180) (size 2.032 1.7272) (drill 1.016) (layers *.Cu *.Mask F.SilkS) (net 34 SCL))
  (pad 5 thru_hole oval (at 0 10.16 180) (size 2.032 1.7272) (drill 1.016) (layers *.Cu *.Mask F.SilkS) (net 35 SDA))
  (pad 6 thru_hole oval (at 0 12.7 180) (size 2.032 1.7272) (drill 1.016) (layers *.Cu *.Mask F.SilkS) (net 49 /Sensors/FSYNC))
  (pad 7 thru_hole oval (at 0 15.24 180) (size 2.032 1.7272) (drill 1.016) (layers *.Cu *.Mask F.SilkS) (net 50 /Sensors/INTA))
  (pad 8 thru_hole oval (at 0 17.78 180) (size 2.032 1.7272) (drill 1.016) (layers *.Cu *.Mask F.SilkS) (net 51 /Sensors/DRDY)))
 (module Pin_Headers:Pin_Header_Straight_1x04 (layer F.Cu) (at 64 110)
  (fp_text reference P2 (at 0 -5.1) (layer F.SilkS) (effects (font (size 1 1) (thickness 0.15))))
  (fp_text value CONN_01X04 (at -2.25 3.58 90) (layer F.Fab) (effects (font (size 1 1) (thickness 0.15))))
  (pad 1 thru_hole rect (at 0 0) (size 2.032 1.7272) (drill 1.016) (layers *.Cu *.Mask F.SilkS) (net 26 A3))
  (pad 2 thru_hole oval (at 0 2.54) (size 2.032 1.7272) (drill 1.016) (layers *.Cu *.Mask F.SilkS) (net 27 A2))
  (pad 3 thru_hole oval (at 0 5.08) (size 2.032 1.7272) (drill 1.016) (layers *.Cu *.Mask F.SilkS) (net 28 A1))
  (pad 4 thru_hole oval (at 0 7.62) (size 2.032 1.7272) (drill 1.016) (layers *.Cu *.Mask F.SilkS) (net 29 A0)))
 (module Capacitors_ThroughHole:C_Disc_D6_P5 (layer F.Cu) (at 70.5 109.5)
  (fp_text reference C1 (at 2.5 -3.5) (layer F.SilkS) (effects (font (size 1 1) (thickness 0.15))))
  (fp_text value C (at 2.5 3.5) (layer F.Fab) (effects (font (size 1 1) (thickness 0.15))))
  (pad 1 thru_hole rect (at 0 0) (size 1.4 1.4) (drill 0.9) (layers *.Cu *.Mask F.SilkS) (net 25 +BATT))
  (pad 2 thru_hole circle (at 5 0) (size 1.4 1.4) (drill 0.9) (layers *.Cu *.Mask F.SilkS) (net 14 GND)))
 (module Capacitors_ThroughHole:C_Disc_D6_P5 (layer F.Cu) (at 217.5 112.25)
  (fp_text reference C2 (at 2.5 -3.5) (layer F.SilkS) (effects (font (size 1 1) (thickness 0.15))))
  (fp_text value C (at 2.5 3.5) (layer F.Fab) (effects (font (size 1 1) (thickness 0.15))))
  (pad 1 thru_hole rect (at 0 0) (size 1.4 1.4) (drill 0.9) (layers *.Cu *.Mask F.SilkS) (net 25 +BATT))
  (pad 2 thru_hole circle (at 5 0) (size 1.4 1.4) (drill 0.9) (layers *.Cu *.Mask F.SilkS) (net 14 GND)))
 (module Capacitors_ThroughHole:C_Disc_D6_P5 (layer F.Cu) (at 165 43.5)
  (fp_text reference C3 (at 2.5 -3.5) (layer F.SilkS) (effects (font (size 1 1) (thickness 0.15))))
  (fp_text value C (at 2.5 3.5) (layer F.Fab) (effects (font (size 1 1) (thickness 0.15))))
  (pad 1 thru_hole rect (at 0 0) (size 1.4 1.4) (drill 0.9) (layers *.Cu *.Mask F.SilkS) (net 25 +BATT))
  (pad 2 thru_hole circle (at 5 0) (size 1.4 1.4) (drill 0.9) (layers *.Cu *.Mask F.SilkS) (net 14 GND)))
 (gr_arc (start 250.25 142) (end 240.25 142) (angle 90) (layer Edge.Cuts) (width 0.15))
 (gr_circle (center 109.25 132.25) (end 110.25 132.25) (layer Edge.Cuts) (width 0.15))
 (gr_circle (center 181 66) (end 182 66) (layer Edge.Cuts) (width 0.15))
 (gr_circle (center 258.5 133.25) (end 259.5 133.25) (layer Edge.Cuts) (width 0.15))
 (gr_circle (center 241.5 150.25) (end 242.5 150.25) (layer Edge.Cuts) (width 0.15))
 (gr_circle (center 164 83) (end 165 83) (layer Edge.Cuts) (width 0.15))
 (gr_circle (center 92.25 149.25) (end 93.25 149.25) (layer Edge.Cuts) (width 0.15))
 (gr_circle (center 63.5 103.5) (end 65.25 103.5) (layer Edge.Cuts) (width 0.15))
 (gr_circle (center 108.5 103.5) (end 110.25 103.5) (layer Edge.Cuts) (width 0.15))
 (gr_circle (center 63.5 148.5) (end 65.25 148.5) (layer Edge.Cuts) (width 0.15))
 (gr_circle (center 135.25 82.25) (end 137 82.25) (layer Edge.Cuts) (width 0.15))
 (gr_circle (center 180.25 37.25) (end 182 37.25) (layer Edge.Cuts) (width 0.15))
 (gr_circle (center 135.25 37.25) (end 137 37.25) (layer Edge.Cuts) (width 0.15))
 (gr_circle (center 212.75 104.5) (end 214.5 104.5) (layer Edge.Cuts) (width 0.15))
 (gr_circle (center 257.75 104.5) (end 259.5 104.5) (layer Edge.Cuts) (width 0.15))
 (gr_circle (center 212.75 149.5) (end 214.5 149.5) (layer Edge.Cuts) (width 0.15))
 (gr_circle (center 140 174.25) (end 141 174.25) (layer Edge.Cuts) (width 0.15))
 (gr_circle (center 128 173.5) (end 129.75 173.5) (layer Edge.Cuts) (width 0.15))
 (gr_line (start 172.75 84.75) (end 132.75 84.75) (layer Edge.Cuts) (width 0.15))
 (gr_line (start 182.75 74.75) (end 182.75 34.75) (layer Edge.Cuts) (width 0.15))
 (gr_line (start 111 101) (end 111 141) (layer Edge.Cuts) (width 0.15))
 (gr_line (start 101 151) (end 61 151) (layer Edge.Cuts) (width 0.15))
 (gr_arc (start 172.75 74.75) (end 172.75 64.75) (angle 90) (layer Edge.Cuts) (width 0.15))
 (gr_arc (start 101 141) (end 101 131) (angle 90) (layer Edge.Cuts) (width 0.15))
 (gr_arc (start 172.75 74.75) (end 162.75 74.75) (angle 90) (layer Edge.Cuts) (width 0.15))
 (gr_arc (start 172.75 74.75) (end 172.75 84.75) (angle 90) (layer Edge.Cuts) (width 0.15))
 (gr_arc (start 101 141) (end 101 131) (angle 90) (layer Edge.Cuts) (width 0.15))
 (gr_arc (start 101 141) (end 91 141) (angle 90) (layer Edge.Cuts) (width 0.15))
 (gr_arc (start 101 141) (end 101 151) (angle 90) (layer Edge.Cuts) (width 0.15))
 (gr_line (start 260.25 142) (end 260.25 102) (layer Edge.Cuts) (width 0.15))
 (gr_line (start 250.25 152) (end 210.25 152) (layer Edge.Cuts) (width 0.15))
 (gr_arc (start 250.25 142) (end 250.25 132) (angle 90) (layer Edge.Cuts) (width 0.15))
 (gr_arc (start 250.25 142) (end 250.25 152) (angle 90) (layer Edge.Cuts) (width 0.15))
 (gr_line (start 210.25 152) (end 210.25 102) (layer Edge.Cuts) (width 0.15))
 (gr_line (start 210.25 102) (end 260.25 102) (layer Edge.Cuts) (width 0.15))
 (gr_line (start 61 151) (end 61 101) (layer Edge.Cuts) (width 0.15))
 (gr_line (start 61 101) (end 111 101) (layer Edge.Cuts) (width 0.15))
 (gr_line (start 132.75 84.75) (end 132.75 84.25) (layer Edge.Cuts) (width 0.15))
 (gr_line (start 132.75 34.75) (end 132.75 84.25) (layer Edge.Cuts) (width 0.15))
 (gr_line (start 182.75 34.75) (end 132.75 34.75) (layer Edge.Cuts) (width 0.15))
 (segment (start 136.266 67.26) (end 135 67.26) (width 0.25) (layer F.Cu) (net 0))
 (segment (start 175.42 37.1524) (end 175.42 37) (width 0.25) (layer F.Cu) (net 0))
 (segment (start 135 77.42) (end 135.1524 77.42) (width 0.25) (layer F.Cu) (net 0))
 (segment (start 154.75 48.5) (end 154.75 40.75) (width 0.25) (layer F.Cu) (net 14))
 (segment (start 156.75 49.75) (end 156 49.75) (width 0.25) (layer F.Cu) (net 14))
 (segment (start 156 49.75) (end 154.75 48.5) (width 0.25) (layer F.Cu) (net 14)))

